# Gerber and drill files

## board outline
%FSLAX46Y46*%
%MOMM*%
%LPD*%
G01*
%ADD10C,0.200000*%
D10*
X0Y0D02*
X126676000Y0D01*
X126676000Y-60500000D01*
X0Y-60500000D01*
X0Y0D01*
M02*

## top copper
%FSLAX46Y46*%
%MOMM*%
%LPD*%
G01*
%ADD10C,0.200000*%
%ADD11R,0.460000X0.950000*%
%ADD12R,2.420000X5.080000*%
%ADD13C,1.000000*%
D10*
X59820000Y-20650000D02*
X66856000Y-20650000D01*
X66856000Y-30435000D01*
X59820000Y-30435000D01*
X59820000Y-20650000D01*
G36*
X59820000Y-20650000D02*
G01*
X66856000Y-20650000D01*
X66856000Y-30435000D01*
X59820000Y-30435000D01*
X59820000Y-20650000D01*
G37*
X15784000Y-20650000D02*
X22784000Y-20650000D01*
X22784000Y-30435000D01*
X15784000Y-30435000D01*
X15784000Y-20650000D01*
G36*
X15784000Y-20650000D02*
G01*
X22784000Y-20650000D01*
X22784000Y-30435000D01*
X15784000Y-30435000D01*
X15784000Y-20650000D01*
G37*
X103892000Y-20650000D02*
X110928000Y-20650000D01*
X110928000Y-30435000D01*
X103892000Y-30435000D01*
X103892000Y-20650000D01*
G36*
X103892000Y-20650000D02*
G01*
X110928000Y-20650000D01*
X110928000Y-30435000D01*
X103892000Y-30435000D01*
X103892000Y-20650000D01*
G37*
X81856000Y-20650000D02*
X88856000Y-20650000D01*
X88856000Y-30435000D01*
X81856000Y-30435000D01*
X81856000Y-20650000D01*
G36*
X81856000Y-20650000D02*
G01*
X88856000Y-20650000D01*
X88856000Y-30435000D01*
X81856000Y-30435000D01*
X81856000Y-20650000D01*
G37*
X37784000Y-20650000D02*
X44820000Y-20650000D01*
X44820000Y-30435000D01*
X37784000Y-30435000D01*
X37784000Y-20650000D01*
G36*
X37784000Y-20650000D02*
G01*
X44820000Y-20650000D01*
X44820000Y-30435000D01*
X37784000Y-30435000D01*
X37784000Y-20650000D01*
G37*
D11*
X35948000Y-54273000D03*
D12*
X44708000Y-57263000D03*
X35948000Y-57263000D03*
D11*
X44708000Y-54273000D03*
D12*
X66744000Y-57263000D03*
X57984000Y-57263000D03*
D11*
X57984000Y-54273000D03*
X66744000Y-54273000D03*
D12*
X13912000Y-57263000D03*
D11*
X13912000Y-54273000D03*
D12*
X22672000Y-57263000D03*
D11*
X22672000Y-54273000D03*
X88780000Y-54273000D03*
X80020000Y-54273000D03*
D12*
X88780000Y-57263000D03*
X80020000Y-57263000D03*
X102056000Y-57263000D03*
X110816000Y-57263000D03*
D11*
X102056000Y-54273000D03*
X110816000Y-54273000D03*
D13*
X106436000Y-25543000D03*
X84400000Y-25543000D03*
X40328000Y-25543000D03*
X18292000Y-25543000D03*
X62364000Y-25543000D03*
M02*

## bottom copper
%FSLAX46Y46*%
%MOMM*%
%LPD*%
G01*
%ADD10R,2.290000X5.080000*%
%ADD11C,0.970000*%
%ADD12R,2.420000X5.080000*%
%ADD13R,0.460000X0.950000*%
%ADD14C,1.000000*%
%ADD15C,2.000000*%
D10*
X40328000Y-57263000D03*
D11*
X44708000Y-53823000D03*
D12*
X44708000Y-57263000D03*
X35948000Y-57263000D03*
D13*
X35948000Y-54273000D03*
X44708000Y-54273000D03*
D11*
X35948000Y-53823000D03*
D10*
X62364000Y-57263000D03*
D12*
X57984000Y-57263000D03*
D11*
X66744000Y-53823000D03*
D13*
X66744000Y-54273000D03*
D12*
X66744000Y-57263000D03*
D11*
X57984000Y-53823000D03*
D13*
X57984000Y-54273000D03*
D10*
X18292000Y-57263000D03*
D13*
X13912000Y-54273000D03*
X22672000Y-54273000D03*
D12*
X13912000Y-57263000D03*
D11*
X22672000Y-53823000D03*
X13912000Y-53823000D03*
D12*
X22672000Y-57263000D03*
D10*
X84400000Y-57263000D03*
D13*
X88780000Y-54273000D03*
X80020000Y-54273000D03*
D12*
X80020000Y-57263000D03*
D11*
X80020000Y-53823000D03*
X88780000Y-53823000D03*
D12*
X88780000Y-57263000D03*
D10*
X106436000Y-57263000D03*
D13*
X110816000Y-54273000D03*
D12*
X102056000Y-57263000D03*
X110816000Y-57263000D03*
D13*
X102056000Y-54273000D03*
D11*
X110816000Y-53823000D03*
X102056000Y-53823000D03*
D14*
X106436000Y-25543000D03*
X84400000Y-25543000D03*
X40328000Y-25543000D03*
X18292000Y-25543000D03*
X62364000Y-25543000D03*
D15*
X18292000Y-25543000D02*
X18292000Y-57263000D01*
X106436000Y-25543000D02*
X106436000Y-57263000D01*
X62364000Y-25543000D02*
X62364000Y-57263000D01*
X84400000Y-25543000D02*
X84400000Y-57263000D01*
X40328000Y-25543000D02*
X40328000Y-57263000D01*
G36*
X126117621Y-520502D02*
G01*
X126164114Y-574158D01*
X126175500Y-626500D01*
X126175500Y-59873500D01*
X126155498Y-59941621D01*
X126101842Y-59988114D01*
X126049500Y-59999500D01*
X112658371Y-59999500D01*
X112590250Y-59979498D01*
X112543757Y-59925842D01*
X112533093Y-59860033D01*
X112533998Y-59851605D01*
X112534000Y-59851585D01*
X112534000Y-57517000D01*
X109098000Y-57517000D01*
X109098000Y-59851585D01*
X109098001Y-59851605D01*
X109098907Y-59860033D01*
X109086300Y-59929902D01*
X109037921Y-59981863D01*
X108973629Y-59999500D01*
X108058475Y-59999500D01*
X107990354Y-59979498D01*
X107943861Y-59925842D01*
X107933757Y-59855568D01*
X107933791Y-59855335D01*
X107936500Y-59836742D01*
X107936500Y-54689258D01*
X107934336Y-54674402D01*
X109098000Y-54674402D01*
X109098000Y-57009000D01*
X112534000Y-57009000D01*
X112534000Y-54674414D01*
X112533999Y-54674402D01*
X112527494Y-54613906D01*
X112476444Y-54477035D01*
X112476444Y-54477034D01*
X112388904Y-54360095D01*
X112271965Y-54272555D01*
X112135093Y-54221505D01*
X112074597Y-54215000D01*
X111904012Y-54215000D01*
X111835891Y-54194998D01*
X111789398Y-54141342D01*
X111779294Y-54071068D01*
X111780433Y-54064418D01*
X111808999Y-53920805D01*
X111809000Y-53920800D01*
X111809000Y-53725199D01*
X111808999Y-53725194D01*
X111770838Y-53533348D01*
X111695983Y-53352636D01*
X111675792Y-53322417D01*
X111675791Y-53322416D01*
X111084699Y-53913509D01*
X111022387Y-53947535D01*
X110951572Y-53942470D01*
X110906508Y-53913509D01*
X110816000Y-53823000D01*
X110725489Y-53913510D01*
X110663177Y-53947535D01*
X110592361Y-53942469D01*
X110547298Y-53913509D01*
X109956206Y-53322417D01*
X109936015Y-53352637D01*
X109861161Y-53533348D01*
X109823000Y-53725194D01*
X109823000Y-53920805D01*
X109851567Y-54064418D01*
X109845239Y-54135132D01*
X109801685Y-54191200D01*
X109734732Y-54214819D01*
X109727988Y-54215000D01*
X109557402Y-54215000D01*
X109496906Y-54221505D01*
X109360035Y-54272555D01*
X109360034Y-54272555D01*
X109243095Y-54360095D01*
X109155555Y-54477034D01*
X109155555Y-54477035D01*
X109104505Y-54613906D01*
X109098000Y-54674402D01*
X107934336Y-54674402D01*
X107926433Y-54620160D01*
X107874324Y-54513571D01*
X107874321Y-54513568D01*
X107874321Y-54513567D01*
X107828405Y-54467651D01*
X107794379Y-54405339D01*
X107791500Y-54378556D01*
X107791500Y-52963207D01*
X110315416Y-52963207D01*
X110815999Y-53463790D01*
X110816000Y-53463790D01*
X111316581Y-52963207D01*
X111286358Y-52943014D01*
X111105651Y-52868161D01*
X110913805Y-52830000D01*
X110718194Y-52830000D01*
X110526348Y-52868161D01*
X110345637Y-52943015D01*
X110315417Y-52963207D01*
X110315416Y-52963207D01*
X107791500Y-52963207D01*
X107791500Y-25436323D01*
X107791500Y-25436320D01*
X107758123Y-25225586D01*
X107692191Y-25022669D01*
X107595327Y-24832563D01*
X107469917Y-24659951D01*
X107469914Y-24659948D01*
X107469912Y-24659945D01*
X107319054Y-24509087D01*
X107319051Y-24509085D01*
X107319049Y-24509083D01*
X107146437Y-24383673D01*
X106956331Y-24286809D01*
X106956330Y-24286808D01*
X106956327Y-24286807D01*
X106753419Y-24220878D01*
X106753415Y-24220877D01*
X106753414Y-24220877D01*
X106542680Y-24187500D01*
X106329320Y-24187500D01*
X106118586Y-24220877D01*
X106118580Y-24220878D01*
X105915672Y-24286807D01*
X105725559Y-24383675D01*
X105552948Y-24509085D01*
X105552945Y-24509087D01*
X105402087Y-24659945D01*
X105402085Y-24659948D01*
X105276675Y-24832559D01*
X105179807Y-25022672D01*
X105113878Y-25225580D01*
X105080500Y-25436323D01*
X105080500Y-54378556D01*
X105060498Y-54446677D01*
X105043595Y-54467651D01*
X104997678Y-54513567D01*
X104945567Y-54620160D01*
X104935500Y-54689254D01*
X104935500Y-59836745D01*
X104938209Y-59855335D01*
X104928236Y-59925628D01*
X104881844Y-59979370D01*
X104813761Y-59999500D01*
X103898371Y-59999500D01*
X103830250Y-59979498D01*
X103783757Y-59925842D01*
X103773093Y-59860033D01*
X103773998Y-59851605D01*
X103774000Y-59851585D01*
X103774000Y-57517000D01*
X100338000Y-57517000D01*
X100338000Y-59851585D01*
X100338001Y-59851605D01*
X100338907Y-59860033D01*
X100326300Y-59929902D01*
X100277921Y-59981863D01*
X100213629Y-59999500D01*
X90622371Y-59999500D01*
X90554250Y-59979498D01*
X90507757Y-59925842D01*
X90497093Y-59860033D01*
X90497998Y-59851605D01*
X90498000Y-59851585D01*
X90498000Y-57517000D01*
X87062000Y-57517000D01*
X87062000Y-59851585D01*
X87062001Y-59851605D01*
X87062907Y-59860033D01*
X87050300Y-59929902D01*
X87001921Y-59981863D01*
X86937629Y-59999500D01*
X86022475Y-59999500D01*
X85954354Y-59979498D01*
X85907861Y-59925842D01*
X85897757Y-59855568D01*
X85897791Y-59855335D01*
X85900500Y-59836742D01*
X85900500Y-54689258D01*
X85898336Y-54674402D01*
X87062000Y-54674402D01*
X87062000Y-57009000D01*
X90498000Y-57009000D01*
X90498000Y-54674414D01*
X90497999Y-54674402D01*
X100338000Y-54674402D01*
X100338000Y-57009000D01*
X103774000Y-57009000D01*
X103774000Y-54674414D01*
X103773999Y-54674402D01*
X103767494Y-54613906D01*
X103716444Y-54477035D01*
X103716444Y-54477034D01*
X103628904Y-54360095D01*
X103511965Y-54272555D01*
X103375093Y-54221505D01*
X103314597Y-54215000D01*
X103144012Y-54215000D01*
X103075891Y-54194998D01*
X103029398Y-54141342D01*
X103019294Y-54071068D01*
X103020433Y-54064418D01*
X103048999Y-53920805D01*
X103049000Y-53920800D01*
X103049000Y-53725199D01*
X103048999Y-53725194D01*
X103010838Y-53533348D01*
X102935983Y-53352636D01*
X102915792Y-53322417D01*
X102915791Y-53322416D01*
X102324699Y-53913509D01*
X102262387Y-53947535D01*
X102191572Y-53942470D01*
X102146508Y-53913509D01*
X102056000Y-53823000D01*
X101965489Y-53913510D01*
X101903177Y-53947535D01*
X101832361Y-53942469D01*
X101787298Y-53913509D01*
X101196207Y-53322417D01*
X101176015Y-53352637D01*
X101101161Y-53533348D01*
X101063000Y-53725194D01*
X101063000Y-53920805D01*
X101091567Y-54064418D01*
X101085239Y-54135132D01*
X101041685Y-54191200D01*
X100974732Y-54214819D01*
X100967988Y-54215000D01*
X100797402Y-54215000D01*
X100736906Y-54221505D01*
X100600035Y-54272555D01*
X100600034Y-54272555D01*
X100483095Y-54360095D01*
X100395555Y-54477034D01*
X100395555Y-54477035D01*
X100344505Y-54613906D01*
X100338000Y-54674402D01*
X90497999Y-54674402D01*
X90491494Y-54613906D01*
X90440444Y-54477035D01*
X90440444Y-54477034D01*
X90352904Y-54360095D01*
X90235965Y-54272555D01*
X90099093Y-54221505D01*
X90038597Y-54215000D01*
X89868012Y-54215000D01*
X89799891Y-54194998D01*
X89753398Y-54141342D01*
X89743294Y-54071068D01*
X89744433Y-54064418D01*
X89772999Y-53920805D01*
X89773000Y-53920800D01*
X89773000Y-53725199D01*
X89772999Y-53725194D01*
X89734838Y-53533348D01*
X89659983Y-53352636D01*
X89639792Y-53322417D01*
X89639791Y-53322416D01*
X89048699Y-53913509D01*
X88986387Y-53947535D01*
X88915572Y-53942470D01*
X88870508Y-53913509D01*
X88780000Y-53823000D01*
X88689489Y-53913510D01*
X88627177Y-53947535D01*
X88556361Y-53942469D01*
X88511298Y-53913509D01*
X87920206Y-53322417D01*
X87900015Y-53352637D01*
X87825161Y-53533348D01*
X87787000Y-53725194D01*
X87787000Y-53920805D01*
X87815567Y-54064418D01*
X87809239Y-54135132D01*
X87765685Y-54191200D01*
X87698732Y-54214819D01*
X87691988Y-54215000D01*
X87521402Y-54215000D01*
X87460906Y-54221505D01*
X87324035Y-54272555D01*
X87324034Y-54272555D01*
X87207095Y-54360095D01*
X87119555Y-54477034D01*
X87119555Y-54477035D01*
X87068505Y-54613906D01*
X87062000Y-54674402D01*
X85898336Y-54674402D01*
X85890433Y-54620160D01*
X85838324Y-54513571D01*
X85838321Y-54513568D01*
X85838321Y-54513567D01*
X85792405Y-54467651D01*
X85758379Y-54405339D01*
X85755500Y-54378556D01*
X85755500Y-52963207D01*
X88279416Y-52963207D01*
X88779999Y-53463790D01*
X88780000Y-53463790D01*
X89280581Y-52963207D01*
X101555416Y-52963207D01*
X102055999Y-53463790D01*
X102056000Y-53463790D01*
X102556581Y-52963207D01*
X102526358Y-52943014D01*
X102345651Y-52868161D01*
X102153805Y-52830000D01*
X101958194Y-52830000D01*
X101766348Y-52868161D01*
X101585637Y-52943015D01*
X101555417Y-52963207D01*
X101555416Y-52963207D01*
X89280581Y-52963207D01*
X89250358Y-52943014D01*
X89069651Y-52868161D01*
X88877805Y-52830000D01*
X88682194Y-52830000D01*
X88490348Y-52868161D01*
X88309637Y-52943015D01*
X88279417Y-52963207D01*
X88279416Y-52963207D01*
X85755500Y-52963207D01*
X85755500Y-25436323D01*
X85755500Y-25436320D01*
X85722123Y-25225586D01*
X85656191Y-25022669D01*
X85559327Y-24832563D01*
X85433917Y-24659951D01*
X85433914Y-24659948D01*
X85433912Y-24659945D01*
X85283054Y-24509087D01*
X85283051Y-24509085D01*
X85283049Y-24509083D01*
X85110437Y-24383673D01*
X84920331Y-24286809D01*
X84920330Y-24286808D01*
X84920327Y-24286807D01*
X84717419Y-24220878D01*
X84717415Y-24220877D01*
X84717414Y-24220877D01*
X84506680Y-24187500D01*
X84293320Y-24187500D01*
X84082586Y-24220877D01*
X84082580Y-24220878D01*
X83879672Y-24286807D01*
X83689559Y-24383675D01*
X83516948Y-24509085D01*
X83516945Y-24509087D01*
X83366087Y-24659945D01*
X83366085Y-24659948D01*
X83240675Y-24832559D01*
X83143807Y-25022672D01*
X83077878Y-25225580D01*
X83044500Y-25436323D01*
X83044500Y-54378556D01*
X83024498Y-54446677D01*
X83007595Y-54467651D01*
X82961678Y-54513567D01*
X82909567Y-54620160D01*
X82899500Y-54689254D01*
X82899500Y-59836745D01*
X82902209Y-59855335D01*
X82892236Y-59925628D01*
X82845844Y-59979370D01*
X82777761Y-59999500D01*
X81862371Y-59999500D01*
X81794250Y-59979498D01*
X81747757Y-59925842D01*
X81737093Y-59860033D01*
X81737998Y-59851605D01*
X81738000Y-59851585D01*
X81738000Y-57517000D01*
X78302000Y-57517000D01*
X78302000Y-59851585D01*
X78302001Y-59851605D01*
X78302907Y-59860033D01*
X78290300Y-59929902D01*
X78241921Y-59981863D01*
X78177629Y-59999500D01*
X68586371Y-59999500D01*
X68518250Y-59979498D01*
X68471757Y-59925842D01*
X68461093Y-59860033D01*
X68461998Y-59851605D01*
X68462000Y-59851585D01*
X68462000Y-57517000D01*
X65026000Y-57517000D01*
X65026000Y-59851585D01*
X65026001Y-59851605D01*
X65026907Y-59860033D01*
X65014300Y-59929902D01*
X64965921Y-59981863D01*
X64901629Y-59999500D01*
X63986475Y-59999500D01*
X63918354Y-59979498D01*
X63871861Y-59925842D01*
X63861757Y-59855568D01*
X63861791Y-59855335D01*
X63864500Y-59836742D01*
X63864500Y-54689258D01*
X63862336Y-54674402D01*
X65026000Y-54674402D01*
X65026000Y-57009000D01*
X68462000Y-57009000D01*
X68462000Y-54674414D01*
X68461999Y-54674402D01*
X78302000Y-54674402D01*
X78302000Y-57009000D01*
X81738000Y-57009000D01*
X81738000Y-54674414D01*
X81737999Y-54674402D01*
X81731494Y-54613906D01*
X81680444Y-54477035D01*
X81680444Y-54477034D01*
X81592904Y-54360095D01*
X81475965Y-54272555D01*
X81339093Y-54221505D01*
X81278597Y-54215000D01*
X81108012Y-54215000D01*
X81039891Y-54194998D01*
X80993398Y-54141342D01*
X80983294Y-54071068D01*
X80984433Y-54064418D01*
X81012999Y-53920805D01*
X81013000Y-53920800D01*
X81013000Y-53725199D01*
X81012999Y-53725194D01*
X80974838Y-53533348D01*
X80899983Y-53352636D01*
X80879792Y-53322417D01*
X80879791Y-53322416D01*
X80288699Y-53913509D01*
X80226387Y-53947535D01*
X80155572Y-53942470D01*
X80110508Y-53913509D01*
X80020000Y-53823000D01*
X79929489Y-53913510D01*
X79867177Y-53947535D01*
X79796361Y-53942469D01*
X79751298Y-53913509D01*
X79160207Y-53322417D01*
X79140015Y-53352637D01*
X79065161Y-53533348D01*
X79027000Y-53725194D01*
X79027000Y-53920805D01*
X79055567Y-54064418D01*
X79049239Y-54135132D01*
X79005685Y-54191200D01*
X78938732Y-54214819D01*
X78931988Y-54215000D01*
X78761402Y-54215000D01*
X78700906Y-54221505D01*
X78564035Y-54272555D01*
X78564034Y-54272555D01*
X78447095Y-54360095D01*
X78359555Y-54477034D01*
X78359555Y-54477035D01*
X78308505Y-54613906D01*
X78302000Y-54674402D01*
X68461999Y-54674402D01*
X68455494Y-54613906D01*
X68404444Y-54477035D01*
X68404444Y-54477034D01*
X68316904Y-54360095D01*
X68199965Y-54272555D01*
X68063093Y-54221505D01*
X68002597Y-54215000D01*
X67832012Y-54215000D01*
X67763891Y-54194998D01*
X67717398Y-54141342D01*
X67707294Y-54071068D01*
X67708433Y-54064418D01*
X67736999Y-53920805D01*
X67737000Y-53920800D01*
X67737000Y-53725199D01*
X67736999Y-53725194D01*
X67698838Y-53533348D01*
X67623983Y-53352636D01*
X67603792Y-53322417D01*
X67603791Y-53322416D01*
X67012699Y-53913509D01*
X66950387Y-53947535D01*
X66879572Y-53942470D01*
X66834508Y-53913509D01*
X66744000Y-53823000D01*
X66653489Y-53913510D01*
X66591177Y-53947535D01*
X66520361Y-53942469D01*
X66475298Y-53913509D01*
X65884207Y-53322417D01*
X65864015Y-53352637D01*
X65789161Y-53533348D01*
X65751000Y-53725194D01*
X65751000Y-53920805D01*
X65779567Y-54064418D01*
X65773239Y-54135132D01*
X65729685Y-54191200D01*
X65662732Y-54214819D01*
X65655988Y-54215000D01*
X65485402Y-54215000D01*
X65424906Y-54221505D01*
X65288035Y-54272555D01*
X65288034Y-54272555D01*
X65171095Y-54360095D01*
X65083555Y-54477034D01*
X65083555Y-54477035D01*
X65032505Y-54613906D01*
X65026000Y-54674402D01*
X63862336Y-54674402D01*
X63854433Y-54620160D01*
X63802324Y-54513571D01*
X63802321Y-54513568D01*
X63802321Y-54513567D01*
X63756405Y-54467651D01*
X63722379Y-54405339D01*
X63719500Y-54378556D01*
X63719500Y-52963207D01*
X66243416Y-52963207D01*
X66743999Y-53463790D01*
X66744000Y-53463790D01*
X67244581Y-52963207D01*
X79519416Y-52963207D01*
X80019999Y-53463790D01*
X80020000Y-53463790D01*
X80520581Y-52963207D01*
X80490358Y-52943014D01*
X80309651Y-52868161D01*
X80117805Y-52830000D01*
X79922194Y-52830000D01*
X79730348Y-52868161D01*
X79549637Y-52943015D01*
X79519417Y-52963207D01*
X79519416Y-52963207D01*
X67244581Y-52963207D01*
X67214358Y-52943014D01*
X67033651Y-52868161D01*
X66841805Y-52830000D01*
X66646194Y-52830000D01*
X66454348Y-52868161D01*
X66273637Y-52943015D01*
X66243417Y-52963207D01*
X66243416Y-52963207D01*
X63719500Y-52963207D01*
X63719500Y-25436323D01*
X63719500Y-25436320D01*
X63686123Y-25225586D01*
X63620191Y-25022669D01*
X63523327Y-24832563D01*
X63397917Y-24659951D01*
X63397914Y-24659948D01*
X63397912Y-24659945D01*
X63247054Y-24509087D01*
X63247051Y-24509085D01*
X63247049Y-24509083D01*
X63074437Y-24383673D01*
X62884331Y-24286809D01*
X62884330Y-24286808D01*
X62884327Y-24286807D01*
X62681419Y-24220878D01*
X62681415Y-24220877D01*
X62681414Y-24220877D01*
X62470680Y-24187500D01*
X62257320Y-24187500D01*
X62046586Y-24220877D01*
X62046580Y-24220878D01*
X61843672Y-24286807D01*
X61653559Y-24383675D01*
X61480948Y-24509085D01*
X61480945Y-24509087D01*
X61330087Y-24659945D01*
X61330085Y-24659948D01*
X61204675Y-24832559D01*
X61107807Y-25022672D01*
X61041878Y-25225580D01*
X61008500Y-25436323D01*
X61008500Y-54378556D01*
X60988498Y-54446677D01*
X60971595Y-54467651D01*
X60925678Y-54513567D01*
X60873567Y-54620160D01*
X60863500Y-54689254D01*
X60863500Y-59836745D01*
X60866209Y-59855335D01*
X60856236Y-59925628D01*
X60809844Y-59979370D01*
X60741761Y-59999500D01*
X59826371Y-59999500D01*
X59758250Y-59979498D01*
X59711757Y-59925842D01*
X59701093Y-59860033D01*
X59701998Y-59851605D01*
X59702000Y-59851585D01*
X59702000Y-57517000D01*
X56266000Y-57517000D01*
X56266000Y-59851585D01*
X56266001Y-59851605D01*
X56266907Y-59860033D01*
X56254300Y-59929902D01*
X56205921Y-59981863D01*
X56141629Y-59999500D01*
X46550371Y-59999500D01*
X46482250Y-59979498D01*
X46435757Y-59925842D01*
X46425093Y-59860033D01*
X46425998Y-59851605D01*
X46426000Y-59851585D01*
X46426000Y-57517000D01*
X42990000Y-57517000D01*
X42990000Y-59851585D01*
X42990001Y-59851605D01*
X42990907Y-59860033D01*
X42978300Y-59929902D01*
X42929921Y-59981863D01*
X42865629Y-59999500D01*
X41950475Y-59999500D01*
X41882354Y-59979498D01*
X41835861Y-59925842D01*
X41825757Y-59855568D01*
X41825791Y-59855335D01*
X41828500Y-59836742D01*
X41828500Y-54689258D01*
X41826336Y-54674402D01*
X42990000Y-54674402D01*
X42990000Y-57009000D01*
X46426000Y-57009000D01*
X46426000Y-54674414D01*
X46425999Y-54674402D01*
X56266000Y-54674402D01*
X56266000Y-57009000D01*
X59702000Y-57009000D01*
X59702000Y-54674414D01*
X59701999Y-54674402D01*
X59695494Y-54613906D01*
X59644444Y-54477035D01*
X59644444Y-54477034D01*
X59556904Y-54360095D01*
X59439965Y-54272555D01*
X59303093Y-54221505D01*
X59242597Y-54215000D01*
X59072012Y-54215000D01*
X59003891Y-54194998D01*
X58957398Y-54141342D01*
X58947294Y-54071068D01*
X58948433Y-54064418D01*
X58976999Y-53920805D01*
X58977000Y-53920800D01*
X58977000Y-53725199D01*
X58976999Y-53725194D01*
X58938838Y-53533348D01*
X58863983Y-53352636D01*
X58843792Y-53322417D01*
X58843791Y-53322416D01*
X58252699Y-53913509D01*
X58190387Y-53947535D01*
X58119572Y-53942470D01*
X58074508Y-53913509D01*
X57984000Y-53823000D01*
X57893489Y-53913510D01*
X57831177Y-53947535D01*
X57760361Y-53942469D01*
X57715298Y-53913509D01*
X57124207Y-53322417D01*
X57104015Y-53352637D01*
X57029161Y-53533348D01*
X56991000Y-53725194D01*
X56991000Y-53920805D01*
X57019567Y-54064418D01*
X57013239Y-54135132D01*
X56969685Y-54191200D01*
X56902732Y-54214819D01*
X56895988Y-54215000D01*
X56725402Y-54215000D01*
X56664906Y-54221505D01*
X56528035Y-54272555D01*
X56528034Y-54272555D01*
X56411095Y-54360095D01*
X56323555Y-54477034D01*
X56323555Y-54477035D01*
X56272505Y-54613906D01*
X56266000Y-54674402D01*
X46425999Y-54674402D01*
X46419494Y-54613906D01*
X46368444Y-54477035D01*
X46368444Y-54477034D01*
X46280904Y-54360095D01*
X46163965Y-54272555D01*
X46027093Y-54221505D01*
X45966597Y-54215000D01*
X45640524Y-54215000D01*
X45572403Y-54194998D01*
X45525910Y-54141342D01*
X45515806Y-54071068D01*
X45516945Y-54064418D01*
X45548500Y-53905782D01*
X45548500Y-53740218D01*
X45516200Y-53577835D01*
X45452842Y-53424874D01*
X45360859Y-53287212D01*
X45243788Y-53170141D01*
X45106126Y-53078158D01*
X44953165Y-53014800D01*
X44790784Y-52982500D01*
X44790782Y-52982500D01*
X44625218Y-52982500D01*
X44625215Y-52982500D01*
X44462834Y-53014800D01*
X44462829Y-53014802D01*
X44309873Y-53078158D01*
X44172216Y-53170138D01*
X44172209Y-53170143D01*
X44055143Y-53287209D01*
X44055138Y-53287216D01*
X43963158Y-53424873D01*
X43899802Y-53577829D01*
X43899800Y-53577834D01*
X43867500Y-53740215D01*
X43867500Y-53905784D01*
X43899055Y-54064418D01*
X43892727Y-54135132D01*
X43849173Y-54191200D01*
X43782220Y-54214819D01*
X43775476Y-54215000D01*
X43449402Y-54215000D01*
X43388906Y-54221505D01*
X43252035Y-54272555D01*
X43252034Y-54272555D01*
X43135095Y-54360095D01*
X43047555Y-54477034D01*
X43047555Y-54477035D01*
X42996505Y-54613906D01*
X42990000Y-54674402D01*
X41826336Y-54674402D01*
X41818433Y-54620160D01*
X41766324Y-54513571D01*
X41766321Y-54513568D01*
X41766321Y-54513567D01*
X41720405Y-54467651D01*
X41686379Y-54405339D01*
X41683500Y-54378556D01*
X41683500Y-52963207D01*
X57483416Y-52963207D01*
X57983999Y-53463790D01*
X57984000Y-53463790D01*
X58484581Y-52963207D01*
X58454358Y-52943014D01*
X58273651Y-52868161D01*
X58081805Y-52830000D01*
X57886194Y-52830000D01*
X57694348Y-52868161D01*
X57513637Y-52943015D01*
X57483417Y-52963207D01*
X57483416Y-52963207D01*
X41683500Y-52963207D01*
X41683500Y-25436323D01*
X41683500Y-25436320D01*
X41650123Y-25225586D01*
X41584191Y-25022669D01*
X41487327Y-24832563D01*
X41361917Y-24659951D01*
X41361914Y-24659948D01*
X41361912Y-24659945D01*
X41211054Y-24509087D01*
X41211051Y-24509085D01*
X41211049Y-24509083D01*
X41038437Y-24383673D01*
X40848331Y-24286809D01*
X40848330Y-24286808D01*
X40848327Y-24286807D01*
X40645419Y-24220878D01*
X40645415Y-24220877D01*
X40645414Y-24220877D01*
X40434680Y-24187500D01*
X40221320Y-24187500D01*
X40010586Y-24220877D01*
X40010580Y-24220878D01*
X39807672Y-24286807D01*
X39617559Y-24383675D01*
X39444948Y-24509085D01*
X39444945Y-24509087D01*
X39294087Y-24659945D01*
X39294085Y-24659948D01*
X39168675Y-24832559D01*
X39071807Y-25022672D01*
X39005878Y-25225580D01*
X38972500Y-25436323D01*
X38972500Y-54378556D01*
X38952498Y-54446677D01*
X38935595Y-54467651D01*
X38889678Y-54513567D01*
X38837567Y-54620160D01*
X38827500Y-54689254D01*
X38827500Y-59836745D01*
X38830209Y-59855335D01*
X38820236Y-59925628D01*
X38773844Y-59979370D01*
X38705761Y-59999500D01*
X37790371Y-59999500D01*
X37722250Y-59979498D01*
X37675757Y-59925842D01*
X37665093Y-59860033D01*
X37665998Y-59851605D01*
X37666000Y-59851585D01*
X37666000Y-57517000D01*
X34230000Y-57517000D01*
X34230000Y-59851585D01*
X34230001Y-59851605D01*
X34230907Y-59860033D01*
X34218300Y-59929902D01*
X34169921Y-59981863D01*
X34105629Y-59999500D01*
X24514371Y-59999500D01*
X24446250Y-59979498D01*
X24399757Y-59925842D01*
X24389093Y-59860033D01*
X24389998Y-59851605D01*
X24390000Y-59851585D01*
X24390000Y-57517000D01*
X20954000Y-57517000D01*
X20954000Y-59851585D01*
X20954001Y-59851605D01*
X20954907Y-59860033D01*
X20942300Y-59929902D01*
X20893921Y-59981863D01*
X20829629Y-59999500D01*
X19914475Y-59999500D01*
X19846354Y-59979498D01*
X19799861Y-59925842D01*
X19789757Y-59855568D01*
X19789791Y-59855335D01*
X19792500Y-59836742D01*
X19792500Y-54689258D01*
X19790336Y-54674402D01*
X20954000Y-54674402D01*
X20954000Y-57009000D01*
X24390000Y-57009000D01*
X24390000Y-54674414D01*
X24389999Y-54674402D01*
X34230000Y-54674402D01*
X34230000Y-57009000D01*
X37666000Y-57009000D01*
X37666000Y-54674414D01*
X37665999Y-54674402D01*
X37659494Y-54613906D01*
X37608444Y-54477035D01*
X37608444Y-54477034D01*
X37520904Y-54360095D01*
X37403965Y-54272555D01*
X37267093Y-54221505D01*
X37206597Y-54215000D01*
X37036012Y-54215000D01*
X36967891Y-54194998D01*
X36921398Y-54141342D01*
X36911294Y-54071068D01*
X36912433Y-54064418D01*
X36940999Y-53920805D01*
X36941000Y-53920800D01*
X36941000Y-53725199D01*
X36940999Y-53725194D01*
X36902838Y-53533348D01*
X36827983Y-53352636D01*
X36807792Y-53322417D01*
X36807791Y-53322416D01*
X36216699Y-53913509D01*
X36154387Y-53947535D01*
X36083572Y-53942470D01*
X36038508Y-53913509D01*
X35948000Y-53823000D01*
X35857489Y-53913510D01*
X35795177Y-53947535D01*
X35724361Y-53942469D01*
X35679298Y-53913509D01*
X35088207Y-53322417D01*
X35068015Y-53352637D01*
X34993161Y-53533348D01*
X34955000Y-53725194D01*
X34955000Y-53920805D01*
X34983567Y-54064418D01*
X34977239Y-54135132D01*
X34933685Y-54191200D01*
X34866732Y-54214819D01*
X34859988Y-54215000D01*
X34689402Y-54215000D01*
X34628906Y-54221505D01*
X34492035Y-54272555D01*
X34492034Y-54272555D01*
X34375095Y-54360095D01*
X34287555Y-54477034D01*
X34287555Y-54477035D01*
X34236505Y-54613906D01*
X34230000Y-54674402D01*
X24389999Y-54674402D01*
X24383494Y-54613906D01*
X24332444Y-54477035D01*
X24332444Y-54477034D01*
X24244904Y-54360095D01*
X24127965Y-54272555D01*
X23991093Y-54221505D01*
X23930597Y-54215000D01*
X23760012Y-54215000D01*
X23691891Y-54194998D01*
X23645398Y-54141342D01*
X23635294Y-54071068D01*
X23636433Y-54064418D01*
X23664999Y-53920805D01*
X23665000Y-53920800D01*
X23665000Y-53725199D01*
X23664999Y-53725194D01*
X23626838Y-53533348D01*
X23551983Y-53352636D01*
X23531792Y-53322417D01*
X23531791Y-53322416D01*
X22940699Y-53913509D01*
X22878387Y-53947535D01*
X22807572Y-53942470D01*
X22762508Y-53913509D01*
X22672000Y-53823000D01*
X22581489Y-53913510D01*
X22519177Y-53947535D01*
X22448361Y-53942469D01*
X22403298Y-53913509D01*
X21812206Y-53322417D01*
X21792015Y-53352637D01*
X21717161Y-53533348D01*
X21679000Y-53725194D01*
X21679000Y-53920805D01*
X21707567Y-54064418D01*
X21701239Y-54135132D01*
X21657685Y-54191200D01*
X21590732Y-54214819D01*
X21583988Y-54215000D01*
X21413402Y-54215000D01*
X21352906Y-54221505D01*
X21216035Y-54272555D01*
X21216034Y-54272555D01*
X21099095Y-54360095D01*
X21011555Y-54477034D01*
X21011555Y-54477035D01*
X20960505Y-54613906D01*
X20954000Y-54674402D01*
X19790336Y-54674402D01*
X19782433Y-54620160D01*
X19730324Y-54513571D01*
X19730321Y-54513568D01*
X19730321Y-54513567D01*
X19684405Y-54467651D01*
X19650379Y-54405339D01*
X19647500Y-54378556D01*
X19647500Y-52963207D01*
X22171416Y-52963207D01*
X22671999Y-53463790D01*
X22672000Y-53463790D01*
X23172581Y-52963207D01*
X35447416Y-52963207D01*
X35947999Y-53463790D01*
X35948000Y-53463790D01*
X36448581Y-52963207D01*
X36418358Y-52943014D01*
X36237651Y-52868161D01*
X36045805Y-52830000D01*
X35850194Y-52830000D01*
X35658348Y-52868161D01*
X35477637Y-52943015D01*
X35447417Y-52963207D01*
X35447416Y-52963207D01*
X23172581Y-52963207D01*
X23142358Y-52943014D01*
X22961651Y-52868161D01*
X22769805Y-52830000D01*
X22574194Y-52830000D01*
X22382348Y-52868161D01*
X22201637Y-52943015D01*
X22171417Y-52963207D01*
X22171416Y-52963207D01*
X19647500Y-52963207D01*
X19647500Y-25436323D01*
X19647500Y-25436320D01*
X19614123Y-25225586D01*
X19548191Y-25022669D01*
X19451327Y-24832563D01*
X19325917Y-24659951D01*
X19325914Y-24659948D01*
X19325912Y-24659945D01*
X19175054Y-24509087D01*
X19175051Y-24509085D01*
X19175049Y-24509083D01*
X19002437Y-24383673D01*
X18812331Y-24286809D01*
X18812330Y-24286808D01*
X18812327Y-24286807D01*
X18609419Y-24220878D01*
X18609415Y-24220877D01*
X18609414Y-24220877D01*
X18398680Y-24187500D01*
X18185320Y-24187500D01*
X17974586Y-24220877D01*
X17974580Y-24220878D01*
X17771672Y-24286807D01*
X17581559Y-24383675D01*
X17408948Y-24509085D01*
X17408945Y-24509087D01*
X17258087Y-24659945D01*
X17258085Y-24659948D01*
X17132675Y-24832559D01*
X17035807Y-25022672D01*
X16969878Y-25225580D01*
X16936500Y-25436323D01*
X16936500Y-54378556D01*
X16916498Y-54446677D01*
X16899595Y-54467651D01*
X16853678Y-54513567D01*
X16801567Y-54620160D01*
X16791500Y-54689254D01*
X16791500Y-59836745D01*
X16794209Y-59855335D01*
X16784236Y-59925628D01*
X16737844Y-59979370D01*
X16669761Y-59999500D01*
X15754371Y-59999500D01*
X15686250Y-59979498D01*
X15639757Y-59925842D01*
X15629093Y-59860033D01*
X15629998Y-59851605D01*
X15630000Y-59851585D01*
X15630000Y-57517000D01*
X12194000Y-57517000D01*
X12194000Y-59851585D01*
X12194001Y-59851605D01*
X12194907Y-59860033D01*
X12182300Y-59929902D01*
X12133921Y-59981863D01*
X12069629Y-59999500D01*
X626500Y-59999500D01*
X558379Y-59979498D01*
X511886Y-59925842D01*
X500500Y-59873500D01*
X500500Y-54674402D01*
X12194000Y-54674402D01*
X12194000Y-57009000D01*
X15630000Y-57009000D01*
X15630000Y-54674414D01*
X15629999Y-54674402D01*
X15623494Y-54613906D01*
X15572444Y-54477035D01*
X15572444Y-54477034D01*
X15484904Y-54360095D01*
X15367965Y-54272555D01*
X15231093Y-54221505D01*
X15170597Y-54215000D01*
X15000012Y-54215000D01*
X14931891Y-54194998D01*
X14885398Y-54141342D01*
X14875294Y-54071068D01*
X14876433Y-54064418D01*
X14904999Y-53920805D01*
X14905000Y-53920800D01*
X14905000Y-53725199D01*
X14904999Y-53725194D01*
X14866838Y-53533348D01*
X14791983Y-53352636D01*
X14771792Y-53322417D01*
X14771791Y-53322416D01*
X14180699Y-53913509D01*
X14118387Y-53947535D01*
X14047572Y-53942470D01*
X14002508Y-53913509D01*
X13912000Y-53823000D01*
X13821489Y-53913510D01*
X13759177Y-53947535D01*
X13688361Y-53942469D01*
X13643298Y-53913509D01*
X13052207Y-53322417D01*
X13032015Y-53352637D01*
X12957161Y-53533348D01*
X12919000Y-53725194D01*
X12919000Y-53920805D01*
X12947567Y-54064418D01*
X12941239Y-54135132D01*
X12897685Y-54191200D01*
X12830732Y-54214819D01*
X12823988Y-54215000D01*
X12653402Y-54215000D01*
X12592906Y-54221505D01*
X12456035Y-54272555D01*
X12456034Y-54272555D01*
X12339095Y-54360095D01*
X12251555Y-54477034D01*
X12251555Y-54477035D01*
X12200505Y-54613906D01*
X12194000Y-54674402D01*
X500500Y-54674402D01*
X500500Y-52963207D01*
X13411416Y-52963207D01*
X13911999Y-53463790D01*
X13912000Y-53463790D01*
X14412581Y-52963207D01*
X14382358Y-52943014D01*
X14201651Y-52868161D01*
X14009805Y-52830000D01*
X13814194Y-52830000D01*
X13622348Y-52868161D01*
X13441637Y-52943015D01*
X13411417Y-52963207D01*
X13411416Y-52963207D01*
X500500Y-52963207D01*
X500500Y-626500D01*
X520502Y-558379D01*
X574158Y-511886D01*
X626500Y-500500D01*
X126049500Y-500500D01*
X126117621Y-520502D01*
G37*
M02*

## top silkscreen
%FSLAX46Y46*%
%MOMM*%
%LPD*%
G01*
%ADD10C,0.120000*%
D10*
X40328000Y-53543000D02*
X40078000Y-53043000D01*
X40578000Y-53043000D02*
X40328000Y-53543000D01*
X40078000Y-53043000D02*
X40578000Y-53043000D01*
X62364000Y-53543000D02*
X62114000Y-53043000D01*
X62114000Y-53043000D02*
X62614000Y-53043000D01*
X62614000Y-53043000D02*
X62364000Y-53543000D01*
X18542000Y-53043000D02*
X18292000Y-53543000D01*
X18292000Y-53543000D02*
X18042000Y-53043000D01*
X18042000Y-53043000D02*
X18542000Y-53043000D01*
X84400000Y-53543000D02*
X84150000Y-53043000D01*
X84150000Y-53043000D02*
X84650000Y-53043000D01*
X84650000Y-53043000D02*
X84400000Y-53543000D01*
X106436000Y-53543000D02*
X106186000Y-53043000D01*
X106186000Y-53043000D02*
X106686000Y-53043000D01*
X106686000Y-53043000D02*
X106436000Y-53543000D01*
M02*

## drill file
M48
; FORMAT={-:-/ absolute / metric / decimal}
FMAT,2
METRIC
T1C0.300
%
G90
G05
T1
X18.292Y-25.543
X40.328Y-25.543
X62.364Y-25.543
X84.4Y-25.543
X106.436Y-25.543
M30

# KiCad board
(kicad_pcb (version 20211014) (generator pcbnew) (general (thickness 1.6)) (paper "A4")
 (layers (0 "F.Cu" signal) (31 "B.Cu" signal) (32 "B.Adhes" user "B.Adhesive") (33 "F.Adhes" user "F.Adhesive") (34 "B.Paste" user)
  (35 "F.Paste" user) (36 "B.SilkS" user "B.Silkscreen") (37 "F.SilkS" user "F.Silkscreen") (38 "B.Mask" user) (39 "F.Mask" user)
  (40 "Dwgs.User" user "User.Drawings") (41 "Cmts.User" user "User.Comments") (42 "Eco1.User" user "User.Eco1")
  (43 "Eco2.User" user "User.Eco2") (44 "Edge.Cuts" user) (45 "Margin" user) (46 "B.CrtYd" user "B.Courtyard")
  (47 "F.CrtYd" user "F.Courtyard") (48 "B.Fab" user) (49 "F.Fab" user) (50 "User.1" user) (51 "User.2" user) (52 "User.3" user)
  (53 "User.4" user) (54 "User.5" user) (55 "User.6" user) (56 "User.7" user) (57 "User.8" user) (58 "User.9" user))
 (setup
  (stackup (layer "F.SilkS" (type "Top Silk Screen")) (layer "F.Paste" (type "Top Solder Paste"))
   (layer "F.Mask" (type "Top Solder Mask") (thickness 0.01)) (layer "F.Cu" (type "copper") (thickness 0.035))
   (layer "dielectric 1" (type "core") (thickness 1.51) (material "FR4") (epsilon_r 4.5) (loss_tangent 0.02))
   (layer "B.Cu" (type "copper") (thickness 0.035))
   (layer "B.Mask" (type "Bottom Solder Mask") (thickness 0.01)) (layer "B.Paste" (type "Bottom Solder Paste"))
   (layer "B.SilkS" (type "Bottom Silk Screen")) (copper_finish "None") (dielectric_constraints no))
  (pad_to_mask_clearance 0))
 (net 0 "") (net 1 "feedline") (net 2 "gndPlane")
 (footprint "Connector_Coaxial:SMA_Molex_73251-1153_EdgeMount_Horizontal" (layer "F.Cu") (at 40.328 55.543 90)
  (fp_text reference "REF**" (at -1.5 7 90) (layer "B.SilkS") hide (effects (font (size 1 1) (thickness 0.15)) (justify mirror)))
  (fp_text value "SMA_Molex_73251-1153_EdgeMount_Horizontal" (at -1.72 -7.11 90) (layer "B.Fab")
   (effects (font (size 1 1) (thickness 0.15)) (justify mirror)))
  (fp_line (start 2 0) (end 2.5 -0.25) (layer "F.SilkS") (width 0.12))
  (fp_line (start 2.5 0.25) (end 2 0) (layer "F.SilkS") (width 0.12))
  (fp_line (start 2.5 -0.25) (end 2.5 0.25) (layer "F.SilkS") (width 0.12))
  (pad "1" smd rect (at -1.72 0 90) (size 5.08 2.29) (layers "B.Cu" "B.Paste" "B.Mask") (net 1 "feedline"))
  (pad "2" smd rect (at 1.27 -4.38 90) (size 0.95 0.46) (layers "F.Cu"))
  (pad "2" smd circle (at 1.72 4.38 90) (size 0.97 0.97) (layers "B.Cu" "B.Paste" "B.Mask"))
  (pad "2" smd rect (at -1.72 4.38 90) (size 5.08 2.42) (layers "F.Cu" "F.Paste" "F.Mask"))
  (pad "2" smd rect (at -1.72 4.38 90) (size 5.08 2.42) (layers "B.Cu" "B.Paste" "B.Mask") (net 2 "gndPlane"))
  (pad "2" smd rect (at -1.72 -4.38 90) (size 5.08 2.42) (layers "F.Cu" "F.Paste" "F.Mask"))
  (pad "2" smd rect (at -1.72 -4.38 90) (size 5.08 2.42) (layers "B.Cu" "B.Paste" "B.Mask") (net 2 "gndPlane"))
  (pad "2" smd rect (at 1.27 4.38 90) (size 0.95 0.46) (layers "F.Cu"))
  (pad "2" smd rect (at 1.27 -4.38 90) (size 0.95 0.46) (layers "B.Cu" "B.Paste" "B.Mask") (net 2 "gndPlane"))
  (pad "2" smd rect (at 1.27 4.38 90) (size 0.95 0.46) (layers "B.Cu" "B.Paste" "B.Mask") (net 2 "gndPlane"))
  (pad "2" smd circle (at 1.72 -4.38 90) (size 0.97 0.97) (layers "B.Cu" "B.Paste" "B.Mask") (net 2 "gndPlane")))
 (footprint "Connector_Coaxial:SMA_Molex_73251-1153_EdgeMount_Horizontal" (layer "F.Cu") (at 62.364 55.543 90)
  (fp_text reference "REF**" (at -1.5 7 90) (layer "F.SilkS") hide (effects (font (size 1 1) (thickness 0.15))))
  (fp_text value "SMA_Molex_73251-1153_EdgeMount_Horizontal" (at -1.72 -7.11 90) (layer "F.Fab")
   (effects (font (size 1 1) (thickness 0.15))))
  (fp_line (start 2 0) (end 2.5 -0.25) (layer "F.SilkS") (width 0.12))
  (fp_line (start 2.5 -0.25) (end 2.5 0.25) (layer "F.SilkS") (width 0.12))
  (fp_line (start 2.5 0.25) (end 2 0) (layer "F.SilkS") (width 0.12))
  (pad "1" smd rect (at -1.72 0 90) (size 5.08 2.29) (layers "B.Cu" "B.Paste" "B.Mask") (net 1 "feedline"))
  (pad "2" smd rect (at -1.72 4.38 90) (size 5.08 2.42) (layers "F.Cu" "B.Paste" "B.Mask"))
  (pad "2" smd rect (at -1.72 -4.38 90) (size 5.08 2.42) (layers "F.Cu" "F.Paste" "F.Mask"))
  (pad "2" smd rect (at 1.27 -4.38 90) (size 0.95 0.46) (layers "F.Cu"))
  (pad "2" smd rect (at -1.72 -4.38 90) (size 5.08 2.42) (layers "B.Cu" "B.Paste" "B.Mask") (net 2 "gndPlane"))
  (pad "2" smd circle (at 1.72 4.38 90) (size 0.97 0.97) (layers "B.Cu" "B.Paste" "B.Mask") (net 2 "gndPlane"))
  (pad "2" smd rect (at 1.27 4.38 90) (size 0.95 0.46) (layers "F.Cu"))
  (pad "2" smd rect (at 1.27 4.38 90) (size 0.95 0.46) (layers "B.Cu") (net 2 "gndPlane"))
  (pad "2" smd rect (at -1.72 4.38 90) (size 5.08 2.42) (layers "B.Cu" "F.Paste" "F.Mask") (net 2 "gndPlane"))
  (pad "2" smd circle (at 1.72 -4.38 90) (size 0.97 0.97) (layers "B.Cu" "B.Paste" "B.Mask") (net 2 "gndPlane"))
  (pad "2" smd rect (at 1.27 -4.38 90) (size 0.95 0.46) (layers "B.Cu") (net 2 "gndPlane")))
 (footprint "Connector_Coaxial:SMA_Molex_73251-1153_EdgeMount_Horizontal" (layer "F.Cu") (at 18.292 55.543 90)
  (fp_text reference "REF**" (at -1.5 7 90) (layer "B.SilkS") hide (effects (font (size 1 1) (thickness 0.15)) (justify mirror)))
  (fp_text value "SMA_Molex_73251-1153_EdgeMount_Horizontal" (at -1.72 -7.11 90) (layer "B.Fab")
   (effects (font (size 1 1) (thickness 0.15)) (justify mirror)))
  (fp_line (start 2.5 0.25) (end 2 0) (layer "F.SilkS") (width 0.12))
  (fp_line (start 2 0) (end 2.5 -0.25) (layer "F.SilkS") (width 0.12))
  (fp_line (start 2.5 -0.25) (end 2.5 0.25) (layer "F.SilkS") (width 0.12))
  (pad "1" smd rect (at -1.72 0 90) (size 5.08 2.29) (layers "B.Cu" "B.Paste" "B.Mask") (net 1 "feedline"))
  (pad "2" smd rect (at -1.72 -4.38 90) (size 5.08 2.42) (layers "F.Cu" "F.Paste" "F.Mask"))
  (pad "2" smd rect (at 1.27 -4.38 90) (size 0.95 0.46) (layers "B.Cu" "B.Paste" "B.Mask") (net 2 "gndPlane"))
  (pad "2" smd rect (at 1.27 -4.38 90) (size 0.95 0.46) (layers "F.Cu"))
  (pad "2" smd rect (at 1.27 4.38 90) (size 0.95 0.46) (layers "B.Cu") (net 2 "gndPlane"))
  (pad "2" smd rect (at -1.72 -4.38 90) (size 5.08 2.42) (layers "B.Cu" "B.Paste" "B.Mask") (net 2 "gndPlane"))
  (pad "2" smd circle (at 1.72 4.38 90) (size 0.97 0.97) (layers "B.Cu" "B.Paste" "B.Mask") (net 2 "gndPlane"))
  (pad "2" smd rect (at -1.72 4.38 90) (size 5.08 2.42) (layers "F.Cu" "B.Paste" "B.Mask"))
  (pad "2" smd rect (at 1.27 4.38 90) (size 0.95 0.46) (layers "F.Cu"))
  (pad "2" smd circle (at 1.72 -4.38 90) (size 0.97 0.97) (layers "B.Cu" "B.Paste" "B.Mask") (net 2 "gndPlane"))
  (pad "3" smd rect (at -1.72 4.38 90) (size 5.08 2.42) (layers "B.Cu" "F.Paste" "F.Mask") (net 2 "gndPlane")))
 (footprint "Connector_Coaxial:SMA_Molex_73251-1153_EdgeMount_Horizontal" (layer "F.Cu") (at 84.4 55.543 90)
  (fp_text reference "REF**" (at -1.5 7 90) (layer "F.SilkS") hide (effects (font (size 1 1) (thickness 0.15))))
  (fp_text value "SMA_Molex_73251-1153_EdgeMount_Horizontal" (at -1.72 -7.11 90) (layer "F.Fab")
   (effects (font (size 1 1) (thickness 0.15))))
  (fp_line (start 2 0) (end 2.5 -0.25) (layer "F.SilkS") (width 0.12))
  (fp_line (start 2.5 -0.25) (end 2.5 0.25) (layer "F.SilkS") (width 0.12))
  (fp_line (start 2.5 0.25) (end 2 0) (layer "F.SilkS") (width 0.12))
  (pad "1" smd rect (at -1.72 0 90) (size 5.08 2.29) (layers "B.Cu" "B.Paste" "B.Mask") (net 1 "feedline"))
  (pad "2" smd rect (at 1.27 4.38 90) (size 0.95 0.46) (layers "B.Cu") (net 2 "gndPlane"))
  (pad "2" smd rect (at 1.27 4.38 90) (size 0.95 0.46) (layers "F.Cu"))
  (pad "2" smd rect (at 1.27 -4.38 90) (size 0.95 0.46) (layers "F.Cu"))
  (pad "2" smd rect (at 1.27 -4.38 90) (size 0.95 0.46) (layers "B.Cu") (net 2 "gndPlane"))
  (pad "2" smd rect (at -1.72 -4.38 90) (size 5.08 2.42) (layers "B.Cu" "B.Paste" "B.Mask") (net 2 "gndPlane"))
  (pad "2" smd circle (at 1.72 -4.38 90) (size 0.97 0.97) (layers "B.Cu" "B.Paste" "B.Mask") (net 2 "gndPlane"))
  (pad "2" smd rect (at -1.72 4.38 90) (size 5.08 2.42) (layers "F.Cu" "F.Paste" "F.Mask"))
  (pad "2" smd circle (at 1.72 4.38 90) (size 0.97 0.97) (layers "B.Cu" "B.Paste" "B.Mask") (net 2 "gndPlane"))
  (pad "2" smd rect (at -1.72 4.38 90) (size 5.08 2.42) (layers "B.Cu" "B.Paste" "B.Mask") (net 2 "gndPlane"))
  (pad "2" smd rect (at -1.72 -4.38 90) (size 5.08 2.42) (layers "F.Cu" "F.Paste" "F.Mask")))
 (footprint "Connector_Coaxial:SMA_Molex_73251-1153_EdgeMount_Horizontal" (layer "F.Cu") (at 106.436 55.543 90)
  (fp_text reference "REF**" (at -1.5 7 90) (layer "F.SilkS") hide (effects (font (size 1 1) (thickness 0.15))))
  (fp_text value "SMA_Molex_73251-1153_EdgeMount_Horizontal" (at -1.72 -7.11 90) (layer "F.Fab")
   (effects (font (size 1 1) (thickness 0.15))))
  (fp_line (start 2 0) (end 2.5 -0.25) (layer "F.SilkS") (width 0.12))
  (fp_line (start 2.5 -0.25) (end 2.5 0.25) (layer "F.SilkS") (width 0.12))
  (fp_line (start 2.5 0.25) (end 2 0) (layer "F.SilkS") (width 0.12))
  (pad "1" smd rect (at -1.72 0 90) (size 5.08 2.29) (layers "B.Cu" "B.Paste" "B.Mask") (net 1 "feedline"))
  (pad "2" smd rect (at 1.27 4.38 90) (size 0.95 0.46) (layers "B.Cu") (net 2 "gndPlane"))
  (pad "2" smd rect (at -1.72 -4.38 90) (size 5.08 2.42) (layers "B.Cu" "B.Paste" "B.Mask") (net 2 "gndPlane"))
  (pad "2" smd rect (at -1.72 -4.38 90) (size 5.08 2.42) (layers "F.Cu" "F.Paste" "F.Mask"))
  (pad "2" smd rect (at -1.72 4.38 90) (size 5.08 2.42) (layers "B.Cu" "B.Paste" "B.Mask") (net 2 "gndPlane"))
  (pad "2" smd rect (at 1.27 -4.38 90) (size 0.95 0.46) (layers "B.Cu") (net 2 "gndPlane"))
  (pad "2" smd circle (at 1.72 4.38 90) (size 0.97 0.97) (layers "B.Cu" "B.Paste" "B.Mask") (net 2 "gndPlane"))
  (pad "2" smd rect (at -1.72 4.38 90) (size 5.08 2.42) (layers "F.Cu" "F.Paste" "F.Mask"))
  (pad "2" smd circle (at 1.72 -4.38 90) (size 0.97 0.97) (layers "B.Cu" "B.Paste" "B.Mask") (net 2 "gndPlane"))
  (pad "2" smd rect (at 1.27 -4.38 90) (size 0.95 0.46) (layers "F.Cu"))
  (pad "2" smd rect (at 1.27 4.38 90) (size 0.95 0.46) (layers "F.Cu")))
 (gr_rect (start 59.82 20.65) (end 66.856 30.435) (layer "F.Cu") (width 0.2) (fill solid))
 (gr_rect (start 15.784 20.65) (end 22.784 30.435) (layer "F.Cu") (width 0.2) (fill solid))
 (gr_rect (start 103.892 20.65) (end 110.928 30.435) (layer "F.Cu") (width 0.2) (fill solid))
 (gr_rect (start 81.856 20.65) (end 88.856 30.435) (layer "F.Cu") (width 0.2) (fill solid))
 (gr_rect (start 37.784 20.65) (end 44.82 30.435) (layer "F.Cu") (width 0.2) (fill solid))
 (gr_rect (start 0 0) (end 126.676 60.5) (layer "Edge.Cuts") (width 0.2) (fill none))
 (via (at 106.436 25.543) (size 1) (drill 0.3) (layers "F.Cu" "B.Cu") (free) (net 1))
 (via (at 84.4 25.543) (size 1) (drill 0.3) (layers "F.Cu" "B.Cu") (free) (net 1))
 (via (at 40.328 25.543) (size 1) (drill 0.3) (layers "F.Cu" "B.Cu") (free) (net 1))
 (via (at 18.292 25.543) (size 1) (drill 0.3) (layers "F.Cu" "B.Cu") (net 1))
 (via (at 62.364 25.543) (size 1) (drill 0.3) (layers "F.Cu" "B.Cu") (free) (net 1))
 (segment (start 18.292 25.543) (end 18.292 57.263) (width 2) (layer "B.Cu") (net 1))
 (segment (start 106.436 25.543) (end 106.436 57.263) (width 2) (layer "B.Cu") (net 1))
 (segment (start 62.364 25.543) (end 62.364 57.263) (width 2) (layer "B.Cu") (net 1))
 (segment (start 84.4 25.543) (end 84.4 57.263) (width 2) (layer "B.Cu") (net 1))
 (segment (start 40.328 25.543) (end 40.328 57.263) (width 2) (layer "B.Cu") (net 1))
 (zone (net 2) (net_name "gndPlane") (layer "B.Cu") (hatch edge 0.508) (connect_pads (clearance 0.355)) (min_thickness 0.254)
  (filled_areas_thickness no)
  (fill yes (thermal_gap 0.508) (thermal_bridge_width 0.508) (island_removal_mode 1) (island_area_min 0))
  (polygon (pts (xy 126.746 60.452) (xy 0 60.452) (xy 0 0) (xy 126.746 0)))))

